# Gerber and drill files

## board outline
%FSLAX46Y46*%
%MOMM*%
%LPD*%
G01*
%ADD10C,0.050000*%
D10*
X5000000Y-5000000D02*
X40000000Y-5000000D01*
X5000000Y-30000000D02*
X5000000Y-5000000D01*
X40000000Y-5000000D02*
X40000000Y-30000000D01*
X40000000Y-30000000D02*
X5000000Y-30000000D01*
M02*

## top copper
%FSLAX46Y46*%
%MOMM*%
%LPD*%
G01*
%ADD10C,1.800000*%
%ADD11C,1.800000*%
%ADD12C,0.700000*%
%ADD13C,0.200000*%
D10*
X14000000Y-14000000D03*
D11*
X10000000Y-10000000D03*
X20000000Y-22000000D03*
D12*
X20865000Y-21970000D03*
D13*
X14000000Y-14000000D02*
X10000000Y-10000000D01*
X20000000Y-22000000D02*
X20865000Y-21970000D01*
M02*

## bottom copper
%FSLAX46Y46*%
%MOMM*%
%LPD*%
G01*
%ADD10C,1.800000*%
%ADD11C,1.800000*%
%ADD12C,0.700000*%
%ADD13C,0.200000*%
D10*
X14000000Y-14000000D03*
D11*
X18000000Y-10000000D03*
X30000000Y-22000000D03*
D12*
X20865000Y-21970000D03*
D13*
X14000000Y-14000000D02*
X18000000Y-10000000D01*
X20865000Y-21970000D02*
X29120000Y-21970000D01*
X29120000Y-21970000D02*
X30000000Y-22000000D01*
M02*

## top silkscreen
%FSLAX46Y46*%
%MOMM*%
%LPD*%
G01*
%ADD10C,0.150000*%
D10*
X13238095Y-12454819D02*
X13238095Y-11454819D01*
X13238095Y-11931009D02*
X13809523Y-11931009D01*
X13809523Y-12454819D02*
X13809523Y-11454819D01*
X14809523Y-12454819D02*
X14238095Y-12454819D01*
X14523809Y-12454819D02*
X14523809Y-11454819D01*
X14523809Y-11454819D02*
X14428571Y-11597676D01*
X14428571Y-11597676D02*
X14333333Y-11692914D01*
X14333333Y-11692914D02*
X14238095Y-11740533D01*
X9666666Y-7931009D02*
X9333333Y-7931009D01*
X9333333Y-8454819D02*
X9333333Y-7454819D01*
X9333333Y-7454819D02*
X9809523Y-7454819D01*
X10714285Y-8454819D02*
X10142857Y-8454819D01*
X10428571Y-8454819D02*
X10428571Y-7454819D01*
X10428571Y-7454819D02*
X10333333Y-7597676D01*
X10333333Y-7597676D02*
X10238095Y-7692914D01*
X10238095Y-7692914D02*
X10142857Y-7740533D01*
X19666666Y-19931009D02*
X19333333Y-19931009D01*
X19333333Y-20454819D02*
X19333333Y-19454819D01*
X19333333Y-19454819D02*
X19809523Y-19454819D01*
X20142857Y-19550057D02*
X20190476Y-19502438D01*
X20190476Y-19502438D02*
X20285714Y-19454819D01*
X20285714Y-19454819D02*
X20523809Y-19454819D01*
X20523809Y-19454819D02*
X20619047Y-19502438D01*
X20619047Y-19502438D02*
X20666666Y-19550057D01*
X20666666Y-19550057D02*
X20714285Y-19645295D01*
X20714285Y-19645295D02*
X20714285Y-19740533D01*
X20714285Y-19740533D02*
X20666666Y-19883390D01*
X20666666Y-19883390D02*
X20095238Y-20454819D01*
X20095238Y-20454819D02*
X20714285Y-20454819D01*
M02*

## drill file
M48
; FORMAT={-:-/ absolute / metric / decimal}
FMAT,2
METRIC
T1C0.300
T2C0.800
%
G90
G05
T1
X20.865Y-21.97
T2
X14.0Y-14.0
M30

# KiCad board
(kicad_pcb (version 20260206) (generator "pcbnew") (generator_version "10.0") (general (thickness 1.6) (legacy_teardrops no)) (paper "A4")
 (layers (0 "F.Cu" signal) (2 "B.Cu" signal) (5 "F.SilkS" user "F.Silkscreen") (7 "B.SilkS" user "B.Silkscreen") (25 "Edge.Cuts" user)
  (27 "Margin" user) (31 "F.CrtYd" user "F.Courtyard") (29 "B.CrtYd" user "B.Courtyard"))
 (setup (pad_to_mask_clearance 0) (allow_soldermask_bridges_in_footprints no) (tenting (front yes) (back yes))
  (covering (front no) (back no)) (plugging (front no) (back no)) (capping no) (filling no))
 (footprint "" (layer "F.Cu") (at 14 14)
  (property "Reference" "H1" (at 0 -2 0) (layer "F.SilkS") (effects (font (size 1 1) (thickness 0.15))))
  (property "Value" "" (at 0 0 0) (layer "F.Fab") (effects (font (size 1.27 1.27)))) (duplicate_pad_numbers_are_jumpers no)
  (pad "1" thru_hole circle (at 0 0) (size 1.8 1.8) (drill 0.8) (layers "*.Cu" "*.Mask") (remove_unused_layers no) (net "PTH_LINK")))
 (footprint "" (layer "F.Cu") (at 10 10)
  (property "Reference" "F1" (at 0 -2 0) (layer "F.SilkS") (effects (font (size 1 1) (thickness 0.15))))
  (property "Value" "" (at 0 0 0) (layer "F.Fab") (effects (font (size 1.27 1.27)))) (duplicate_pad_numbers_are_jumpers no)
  (pad "1" smd circle (at 0 0) (size 1.8 1.8) (layers "F.Cu" "F.Mask" "F.Paste") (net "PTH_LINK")))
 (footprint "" (layer "F.Cu") (at 20 22)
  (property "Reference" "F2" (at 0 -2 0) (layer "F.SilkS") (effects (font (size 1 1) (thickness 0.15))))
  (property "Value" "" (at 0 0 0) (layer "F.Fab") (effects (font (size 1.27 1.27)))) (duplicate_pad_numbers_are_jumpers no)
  (pad "1" smd circle (at 0 0) (size 1.8 1.8) (layers "F.Cu" "F.Mask" "F.Paste") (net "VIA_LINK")))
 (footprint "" (layer "B.Cu") (at 18 10)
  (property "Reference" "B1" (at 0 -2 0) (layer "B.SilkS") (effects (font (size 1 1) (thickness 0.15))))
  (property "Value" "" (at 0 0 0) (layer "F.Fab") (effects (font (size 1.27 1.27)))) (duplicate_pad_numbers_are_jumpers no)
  (pad "1" smd circle (at 0 0) (size 1.8 1.8) (layers "B.Cu" "B.Mask" "B.Paste") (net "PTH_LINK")))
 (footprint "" (layer "B.Cu") (at 30 22)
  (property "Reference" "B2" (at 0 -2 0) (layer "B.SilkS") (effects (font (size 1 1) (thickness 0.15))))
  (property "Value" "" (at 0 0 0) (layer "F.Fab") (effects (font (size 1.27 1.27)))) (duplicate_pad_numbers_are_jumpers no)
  (pad "1" smd circle (at 0 0) (size 1.8 1.8) (layers "B.Cu" "B.Mask" "B.Paste") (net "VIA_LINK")))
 (gr_line (start 5 5) (end 40 5) (stroke (width 0.05) (type default)) (layer "Edge.Cuts"))
 (gr_line (start 5 30) (end 5 5) (stroke (width 0.05) (type default)) (layer "Edge.Cuts"))
 (gr_line (start 40 5) (end 40 30) (stroke (width 0.05) (type default)) (layer "Edge.Cuts"))
 (gr_line (start 40 30) (end 5 30) (stroke (width 0.05) (type default)) (layer "Edge.Cuts"))
 (segment (start 14 14) (end 10 10) (width 0.2) (layer "F.Cu") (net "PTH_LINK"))
 (segment (start 14 14) (end 18 10) (width 0.2) (layer "B.Cu") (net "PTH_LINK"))
 (segment (start 20 22) (end 20.865 21.97) (width 0.2) (layer "F.Cu") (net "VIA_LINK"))
 (segment (start 20.865 21.97) (end 29.12 21.97) (width 0.2) (layer "B.Cu") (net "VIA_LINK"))
 (segment (start 29.12 21.97) (end 30 22) (width 0.2) (layer "B.Cu") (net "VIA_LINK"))
 (via (at 20.865 21.97) (size 0.7) (drill 0.3) (layers "F.Cu" "B.Cu") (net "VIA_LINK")))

